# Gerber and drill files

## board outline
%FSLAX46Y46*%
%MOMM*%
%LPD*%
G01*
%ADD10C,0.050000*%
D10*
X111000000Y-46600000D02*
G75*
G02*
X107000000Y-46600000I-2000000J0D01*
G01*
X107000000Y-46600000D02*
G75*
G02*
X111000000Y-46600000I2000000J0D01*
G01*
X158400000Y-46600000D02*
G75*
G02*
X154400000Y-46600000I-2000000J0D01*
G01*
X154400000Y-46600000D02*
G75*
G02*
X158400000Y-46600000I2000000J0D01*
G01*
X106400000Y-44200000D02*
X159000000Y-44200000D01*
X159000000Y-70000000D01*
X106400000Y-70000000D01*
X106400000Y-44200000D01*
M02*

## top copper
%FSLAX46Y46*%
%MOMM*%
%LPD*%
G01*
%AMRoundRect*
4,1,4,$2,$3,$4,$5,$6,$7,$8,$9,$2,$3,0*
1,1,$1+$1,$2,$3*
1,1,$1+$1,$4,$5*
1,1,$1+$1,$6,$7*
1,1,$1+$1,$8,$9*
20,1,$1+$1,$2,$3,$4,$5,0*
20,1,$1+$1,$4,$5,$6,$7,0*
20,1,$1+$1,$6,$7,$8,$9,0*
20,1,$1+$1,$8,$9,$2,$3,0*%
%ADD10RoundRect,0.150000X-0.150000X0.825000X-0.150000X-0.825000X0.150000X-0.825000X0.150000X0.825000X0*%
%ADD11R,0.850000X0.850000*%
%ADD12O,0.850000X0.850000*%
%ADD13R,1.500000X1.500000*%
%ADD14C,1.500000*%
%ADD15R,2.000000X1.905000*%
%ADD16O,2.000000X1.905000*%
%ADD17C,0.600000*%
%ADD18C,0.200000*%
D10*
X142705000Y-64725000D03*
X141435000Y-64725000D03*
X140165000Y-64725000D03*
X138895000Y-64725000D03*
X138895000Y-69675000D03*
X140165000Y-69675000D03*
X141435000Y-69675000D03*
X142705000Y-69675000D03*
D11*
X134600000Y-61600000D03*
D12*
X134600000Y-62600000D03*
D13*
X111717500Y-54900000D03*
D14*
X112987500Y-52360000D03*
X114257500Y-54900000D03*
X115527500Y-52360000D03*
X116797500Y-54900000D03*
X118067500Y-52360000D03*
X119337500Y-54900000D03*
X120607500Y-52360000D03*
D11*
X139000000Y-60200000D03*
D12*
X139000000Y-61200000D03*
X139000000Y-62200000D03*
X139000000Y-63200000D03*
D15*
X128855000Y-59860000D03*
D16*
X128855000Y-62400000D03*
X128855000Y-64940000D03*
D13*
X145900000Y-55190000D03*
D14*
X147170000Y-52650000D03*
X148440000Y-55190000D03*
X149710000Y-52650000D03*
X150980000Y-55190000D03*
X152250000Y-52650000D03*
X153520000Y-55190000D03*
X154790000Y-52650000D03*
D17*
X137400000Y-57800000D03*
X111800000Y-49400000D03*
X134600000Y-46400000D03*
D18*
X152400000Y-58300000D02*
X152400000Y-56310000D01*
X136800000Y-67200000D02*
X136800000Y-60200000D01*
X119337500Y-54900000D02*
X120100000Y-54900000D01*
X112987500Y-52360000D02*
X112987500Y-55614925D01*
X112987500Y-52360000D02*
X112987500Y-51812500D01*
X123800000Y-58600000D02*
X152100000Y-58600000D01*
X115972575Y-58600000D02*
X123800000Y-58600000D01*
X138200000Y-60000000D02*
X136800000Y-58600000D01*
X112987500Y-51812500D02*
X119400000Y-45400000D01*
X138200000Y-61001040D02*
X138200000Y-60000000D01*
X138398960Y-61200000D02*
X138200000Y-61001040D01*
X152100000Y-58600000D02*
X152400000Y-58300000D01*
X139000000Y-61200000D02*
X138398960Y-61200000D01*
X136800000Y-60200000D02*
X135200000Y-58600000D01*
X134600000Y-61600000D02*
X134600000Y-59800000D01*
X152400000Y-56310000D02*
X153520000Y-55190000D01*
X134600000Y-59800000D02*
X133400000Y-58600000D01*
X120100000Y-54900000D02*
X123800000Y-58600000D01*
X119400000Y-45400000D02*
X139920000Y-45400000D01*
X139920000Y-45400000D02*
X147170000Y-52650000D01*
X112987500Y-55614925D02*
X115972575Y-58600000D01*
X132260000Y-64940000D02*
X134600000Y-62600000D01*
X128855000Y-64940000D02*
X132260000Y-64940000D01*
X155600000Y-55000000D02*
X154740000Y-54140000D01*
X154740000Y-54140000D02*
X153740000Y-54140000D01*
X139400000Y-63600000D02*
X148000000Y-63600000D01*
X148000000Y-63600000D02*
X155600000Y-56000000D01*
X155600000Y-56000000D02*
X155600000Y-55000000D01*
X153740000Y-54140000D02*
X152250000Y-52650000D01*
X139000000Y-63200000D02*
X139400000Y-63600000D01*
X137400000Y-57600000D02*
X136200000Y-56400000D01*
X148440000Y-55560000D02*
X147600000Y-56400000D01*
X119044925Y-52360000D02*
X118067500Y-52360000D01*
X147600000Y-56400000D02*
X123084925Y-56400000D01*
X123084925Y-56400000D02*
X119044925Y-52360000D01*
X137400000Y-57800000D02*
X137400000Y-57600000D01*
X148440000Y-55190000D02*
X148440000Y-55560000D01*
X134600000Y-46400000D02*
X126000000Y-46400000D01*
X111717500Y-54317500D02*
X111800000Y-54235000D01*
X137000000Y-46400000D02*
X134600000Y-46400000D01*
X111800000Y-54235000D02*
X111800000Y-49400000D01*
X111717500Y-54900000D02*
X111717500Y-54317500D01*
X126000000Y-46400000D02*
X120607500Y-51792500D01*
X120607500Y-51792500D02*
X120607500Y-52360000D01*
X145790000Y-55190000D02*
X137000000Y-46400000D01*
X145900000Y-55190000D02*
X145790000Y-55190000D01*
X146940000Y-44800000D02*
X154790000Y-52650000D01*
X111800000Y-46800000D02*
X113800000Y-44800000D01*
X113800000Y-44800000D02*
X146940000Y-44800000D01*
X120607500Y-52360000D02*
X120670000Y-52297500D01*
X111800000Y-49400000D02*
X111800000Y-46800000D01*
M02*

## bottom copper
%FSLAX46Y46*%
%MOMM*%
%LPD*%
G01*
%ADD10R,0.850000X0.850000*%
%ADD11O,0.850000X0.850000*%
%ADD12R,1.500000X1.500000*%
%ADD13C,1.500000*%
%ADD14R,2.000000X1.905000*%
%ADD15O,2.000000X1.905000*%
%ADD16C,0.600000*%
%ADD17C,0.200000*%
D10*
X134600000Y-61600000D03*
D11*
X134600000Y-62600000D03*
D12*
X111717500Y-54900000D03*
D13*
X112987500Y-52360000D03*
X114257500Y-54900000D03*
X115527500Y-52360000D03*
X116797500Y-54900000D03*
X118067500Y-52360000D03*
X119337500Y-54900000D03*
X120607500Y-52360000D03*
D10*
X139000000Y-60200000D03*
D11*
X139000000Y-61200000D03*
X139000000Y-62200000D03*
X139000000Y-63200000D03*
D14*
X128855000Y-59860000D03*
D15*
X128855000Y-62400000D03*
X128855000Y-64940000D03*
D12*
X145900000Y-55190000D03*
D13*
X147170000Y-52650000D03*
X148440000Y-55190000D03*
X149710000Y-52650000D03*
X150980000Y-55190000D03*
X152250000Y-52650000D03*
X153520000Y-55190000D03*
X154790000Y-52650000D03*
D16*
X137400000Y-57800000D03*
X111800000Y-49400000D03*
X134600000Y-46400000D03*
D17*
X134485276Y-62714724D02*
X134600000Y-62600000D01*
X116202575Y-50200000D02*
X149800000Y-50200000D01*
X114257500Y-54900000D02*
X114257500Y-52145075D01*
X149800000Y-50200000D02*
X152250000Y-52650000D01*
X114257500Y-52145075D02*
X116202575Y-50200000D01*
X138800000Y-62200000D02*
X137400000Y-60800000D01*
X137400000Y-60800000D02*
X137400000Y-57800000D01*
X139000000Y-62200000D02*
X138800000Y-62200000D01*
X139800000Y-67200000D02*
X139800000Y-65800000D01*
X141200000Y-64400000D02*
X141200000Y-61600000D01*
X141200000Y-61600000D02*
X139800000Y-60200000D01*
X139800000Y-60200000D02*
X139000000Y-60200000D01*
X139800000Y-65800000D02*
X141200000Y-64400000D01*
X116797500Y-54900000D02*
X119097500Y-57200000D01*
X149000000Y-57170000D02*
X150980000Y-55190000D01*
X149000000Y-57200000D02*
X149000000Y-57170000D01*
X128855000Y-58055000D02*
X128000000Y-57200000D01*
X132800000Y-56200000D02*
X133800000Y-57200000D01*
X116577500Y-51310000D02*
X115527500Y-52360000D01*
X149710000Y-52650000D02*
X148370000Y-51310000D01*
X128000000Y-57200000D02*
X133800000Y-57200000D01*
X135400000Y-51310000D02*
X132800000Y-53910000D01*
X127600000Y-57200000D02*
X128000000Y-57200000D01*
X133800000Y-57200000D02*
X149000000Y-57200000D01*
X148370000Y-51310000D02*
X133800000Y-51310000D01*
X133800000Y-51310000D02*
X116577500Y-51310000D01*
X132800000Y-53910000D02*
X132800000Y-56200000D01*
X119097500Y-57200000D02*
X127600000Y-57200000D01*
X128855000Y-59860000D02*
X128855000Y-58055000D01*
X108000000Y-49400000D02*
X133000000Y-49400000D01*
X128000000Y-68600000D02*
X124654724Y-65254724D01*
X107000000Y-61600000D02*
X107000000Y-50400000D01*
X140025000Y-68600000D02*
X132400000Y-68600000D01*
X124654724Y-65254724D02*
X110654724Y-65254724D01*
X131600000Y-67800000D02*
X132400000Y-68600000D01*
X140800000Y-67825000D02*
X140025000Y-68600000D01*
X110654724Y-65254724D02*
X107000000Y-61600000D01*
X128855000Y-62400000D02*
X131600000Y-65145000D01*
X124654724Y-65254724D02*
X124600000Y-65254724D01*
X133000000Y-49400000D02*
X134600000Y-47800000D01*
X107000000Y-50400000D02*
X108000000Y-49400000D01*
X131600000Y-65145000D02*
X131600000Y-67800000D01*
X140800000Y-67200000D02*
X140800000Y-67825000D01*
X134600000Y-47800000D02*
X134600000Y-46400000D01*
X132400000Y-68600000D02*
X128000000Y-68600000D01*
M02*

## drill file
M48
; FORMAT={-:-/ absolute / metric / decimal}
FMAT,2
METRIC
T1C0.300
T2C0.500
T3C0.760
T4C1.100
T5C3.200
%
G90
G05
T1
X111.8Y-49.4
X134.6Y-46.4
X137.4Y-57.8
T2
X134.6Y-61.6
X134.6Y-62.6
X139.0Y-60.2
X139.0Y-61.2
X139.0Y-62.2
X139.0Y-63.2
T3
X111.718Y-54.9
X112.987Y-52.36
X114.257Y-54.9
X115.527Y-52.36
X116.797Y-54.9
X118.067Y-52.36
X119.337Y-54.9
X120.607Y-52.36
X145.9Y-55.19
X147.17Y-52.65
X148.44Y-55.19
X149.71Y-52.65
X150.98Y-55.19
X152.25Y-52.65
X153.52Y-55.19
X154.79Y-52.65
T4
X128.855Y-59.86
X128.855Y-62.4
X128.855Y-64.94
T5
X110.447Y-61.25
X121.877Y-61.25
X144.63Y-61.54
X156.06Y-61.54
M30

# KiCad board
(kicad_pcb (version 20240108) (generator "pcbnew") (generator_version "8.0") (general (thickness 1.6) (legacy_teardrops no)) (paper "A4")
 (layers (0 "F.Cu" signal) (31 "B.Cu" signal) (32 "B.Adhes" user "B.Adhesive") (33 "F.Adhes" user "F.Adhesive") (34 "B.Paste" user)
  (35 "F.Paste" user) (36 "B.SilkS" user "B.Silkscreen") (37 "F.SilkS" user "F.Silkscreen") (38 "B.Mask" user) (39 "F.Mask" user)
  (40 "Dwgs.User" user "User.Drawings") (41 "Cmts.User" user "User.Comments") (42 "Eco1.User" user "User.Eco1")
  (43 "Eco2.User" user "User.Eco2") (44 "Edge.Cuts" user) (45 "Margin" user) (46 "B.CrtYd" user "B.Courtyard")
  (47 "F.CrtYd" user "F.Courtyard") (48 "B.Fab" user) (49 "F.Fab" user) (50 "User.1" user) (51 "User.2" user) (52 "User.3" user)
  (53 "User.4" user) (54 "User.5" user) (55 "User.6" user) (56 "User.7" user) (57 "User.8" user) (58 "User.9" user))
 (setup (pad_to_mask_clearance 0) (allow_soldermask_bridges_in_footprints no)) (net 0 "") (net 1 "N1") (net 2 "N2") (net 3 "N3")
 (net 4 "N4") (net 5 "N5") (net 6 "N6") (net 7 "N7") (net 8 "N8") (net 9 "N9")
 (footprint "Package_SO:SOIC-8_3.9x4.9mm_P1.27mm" (layer "F.Cu") (at 140.8 67.2 -90)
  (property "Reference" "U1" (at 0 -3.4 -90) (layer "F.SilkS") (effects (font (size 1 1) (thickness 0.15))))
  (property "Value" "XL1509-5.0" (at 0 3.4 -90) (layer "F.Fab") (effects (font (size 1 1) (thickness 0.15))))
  (pad "1" smd roundrect (at -2.475 -1.905 270) (size 1.95 0.6) (layers "F.Cu" "F.Paste" "F.Mask") (roundrect_rratio 0.25) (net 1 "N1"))
  (pad "2" smd roundrect (at -2.475 -0.635 270) (size 1.95 0.6) (layers "F.Cu" "F.Paste" "F.Mask") (roundrect_rratio 0.25) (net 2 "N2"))
  (pad "3" smd roundrect (at -2.475 0.635 270) (size 1.95 0.6) (layers "F.Cu" "F.Paste" "F.Mask") (roundrect_rratio 0.25) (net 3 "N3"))
  (pad "4" smd roundrect (at -2.475 1.905 270) (size 1.95 0.6) (layers "F.Cu" "F.Paste" "F.Mask") (roundrect_rratio 0.25) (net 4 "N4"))
  (pad "5" smd roundrect (at 2.475 1.905 270) (size 1.95 0.6) (layers "F.Cu" "F.Paste" "F.Mask") (roundrect_rratio 0.25) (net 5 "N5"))
  (pad "6" smd roundrect (at 2.475 0.635 270) (size 1.95 0.6) (layers "F.Cu" "F.Paste" "F.Mask") (roundrect_rratio 0.25))
  (pad "7" smd roundrect (at 2.475 -0.635 270) (size 1.95 0.6) (layers "F.Cu" "F.Paste" "F.Mask") (roundrect_rratio 0.25))
  (pad "8" smd roundrect (at 2.475 -1.905 270) (size 1.95 0.6) (layers "F.Cu" "F.Paste" "F.Mask") (roundrect_rratio 0.25)))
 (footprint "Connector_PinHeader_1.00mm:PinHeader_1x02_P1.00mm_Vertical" (layer "F.Cu") (at 134.6 61.6)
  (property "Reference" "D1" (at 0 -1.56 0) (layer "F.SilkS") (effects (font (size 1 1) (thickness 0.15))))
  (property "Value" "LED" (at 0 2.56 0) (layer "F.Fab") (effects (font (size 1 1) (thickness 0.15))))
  (pad "1" thru_hole rect (at 0 0) (size 0.85 0.85) (drill 0.5) (layers "*.Cu" "*.Mask") (remove_unused_layers no) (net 5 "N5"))
  (pad "2" thru_hole oval (at 0 1) (size 0.85 0.85) (drill 0.5) (layers "*.Cu" "*.Mask") (remove_unused_layers no) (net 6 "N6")))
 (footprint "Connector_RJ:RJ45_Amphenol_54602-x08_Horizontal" (layer "F.Cu") (at 111.7175 54.9)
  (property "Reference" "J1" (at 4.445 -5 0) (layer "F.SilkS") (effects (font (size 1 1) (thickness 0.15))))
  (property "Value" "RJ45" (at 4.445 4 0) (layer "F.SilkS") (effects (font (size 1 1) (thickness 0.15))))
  (pad "" np_thru_hole circle (at -1.27 6.35) (size 3.2 3.2) (drill 3.2) (layers "*.Cu" "*.Mask"))
  (pad "" np_thru_hole circle (at 10.16 6.35) (size 3.2 3.2) (drill 3.2) (layers "*.Cu" "*.Mask"))
  (pad "1" thru_hole rect (at 0 0) (size 1.5 1.5) (drill 0.76) (layers "*.Cu" "*.Mask") (remove_unused_layers no) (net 1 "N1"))
  (pad "2" thru_hole circle (at 1.27 -2.54) (size 1.5 1.5) (drill 0.76) (layers "*.Cu" "*.Mask") (remove_unused_layers no) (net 5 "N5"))
  (pad "3" thru_hole circle (at 2.54 0) (size 1.5 1.5) (drill 0.76) (layers "*.Cu" "*.Mask") (remove_unused_layers no) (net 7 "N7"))
  (pad "4" thru_hole circle (at 3.81 -2.54) (size 1.5 1.5) (drill 0.76) (layers "*.Cu" "*.Mask") (remove_unused_layers no) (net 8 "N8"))
  (pad "5" thru_hole circle (at 5.08 0) (size 1.5 1.5) (drill 0.76) (layers "*.Cu" "*.Mask") (remove_unused_layers no) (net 8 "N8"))
  (pad "6" thru_hole circle (at 6.35 -2.54) (size 1.5 1.5) (drill 0.76) (layers "*.Cu" "*.Mask") (remove_unused_layers no) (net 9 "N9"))
  (pad "7" thru_hole circle (at 7.62 0) (size 1.5 1.5) (drill 0.76) (layers "*.Cu" "*.Mask") (remove_unused_layers no) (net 5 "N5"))
  (pad "8" thru_hole circle (at 8.89 -2.54) (size 1.5 1.5) (drill 0.76) (layers "*.Cu" "*.Mask") (remove_unused_layers no) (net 1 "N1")))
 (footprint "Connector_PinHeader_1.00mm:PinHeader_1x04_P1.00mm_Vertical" (layer "F.Cu") (at 139 60.2)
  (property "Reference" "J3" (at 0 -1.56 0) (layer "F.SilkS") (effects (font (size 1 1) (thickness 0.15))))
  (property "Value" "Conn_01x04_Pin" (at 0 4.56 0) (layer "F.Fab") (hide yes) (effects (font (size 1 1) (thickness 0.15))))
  (pad "1" thru_hole rect (at 0 0) (size 0.85 0.85) (drill 0.5) (layers "*.Cu" "*.Mask") (remove_unused_layers no) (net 2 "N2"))
  (pad "2" thru_hole oval (at 0 1) (size 0.85 0.85) (drill 0.5) (layers "*.Cu" "*.Mask") (remove_unused_layers no) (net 5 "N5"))
  (pad "3" thru_hole oval (at 0 2) (size 0.85 0.85) (drill 0.5) (layers "*.Cu" "*.Mask") (remove_unused_layers no) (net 9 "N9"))
  (pad "4" thru_hole oval (at 0 3) (size 0.85 0.85) (drill 0.5) (layers "*.Cu" "*.Mask") (remove_unused_layers no) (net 7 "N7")))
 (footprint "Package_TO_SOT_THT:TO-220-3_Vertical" (layer "F.Cu") (at 128.855 59.86 -90)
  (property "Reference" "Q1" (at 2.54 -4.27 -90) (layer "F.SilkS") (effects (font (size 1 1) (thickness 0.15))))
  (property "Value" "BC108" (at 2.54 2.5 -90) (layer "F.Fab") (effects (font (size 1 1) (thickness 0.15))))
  (pad "1" thru_hole rect (at 0 0 270) (size 1.905 2) (drill 1.1) (layers "*.Cu" "*.Mask") (remove_unused_layers no) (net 8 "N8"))
  (pad "2" thru_hole oval (at 2.54 0 270) (size 1.905 2) (drill 1.1) (layers "*.Cu" "*.Mask") (remove_unused_layers no) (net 1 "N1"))
  (pad "3" thru_hole oval (at 5.08 0 270) (size 1.905 2) (drill 1.1) (layers "*.Cu" "*.Mask") (remove_unused_layers no) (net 6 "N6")))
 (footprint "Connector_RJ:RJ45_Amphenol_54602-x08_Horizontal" (layer "F.Cu") (at 145.9 55.19)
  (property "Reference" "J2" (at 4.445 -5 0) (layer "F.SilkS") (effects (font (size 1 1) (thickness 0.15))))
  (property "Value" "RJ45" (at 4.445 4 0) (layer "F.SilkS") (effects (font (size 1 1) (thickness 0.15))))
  (pad "" np_thru_hole circle (at -1.27 6.35) (size 3.2 3.2) (drill 3.2) (layers "*.Cu" "*.Mask"))
  (pad "" np_thru_hole circle (at 10.16 6.35) (size 3.2 3.2) (drill 3.2) (layers "*.Cu" "*.Mask"))
  (pad "1" thru_hole rect (at 0 0) (size 1.5 1.5) (drill 0.76) (layers "*.Cu" "*.Mask") (remove_unused_layers no) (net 1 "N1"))
  (pad "2" thru_hole circle (at 1.27 -2.54) (size 1.5 1.5) (drill 0.76) (layers "*.Cu" "*.Mask") (remove_unused_layers no) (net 5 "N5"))
  (pad "3" thru_hole circle (at 2.54 0) (size 1.5 1.5) (drill 0.76) (layers "*.Cu" "*.Mask") (remove_unused_layers no) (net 9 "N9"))
  (pad "4" thru_hole circle (at 3.81 -2.54) (size 1.5 1.5) (drill 0.76) (layers "*.Cu" "*.Mask") (remove_unused_layers no) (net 8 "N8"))
  (pad "5" thru_hole circle (at 5.08 0) (size 1.5 1.5) (drill 0.76) (layers "*.Cu" "*.Mask") (remove_unused_layers no) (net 8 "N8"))
  (pad "6" thru_hole circle (at 6.35 -2.54) (size 1.5 1.5) (drill 0.76) (layers "*.Cu" "*.Mask") (remove_unused_layers no) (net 7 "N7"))
  (pad "7" thru_hole circle (at 7.62 0) (size 1.5 1.5) (drill 0.76) (layers "*.Cu" "*.Mask") (remove_unused_layers no) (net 5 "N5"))
  (pad "8" thru_hole circle (at 8.89 -2.54) (size 1.5 1.5) (drill 0.76) (layers "*.Cu" "*.Mask") (remove_unused_layers no) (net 1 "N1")))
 (gr_circle (center 109 46.6) (end 110.6 47.8) (stroke (width 0.05) (type default)) (fill none) (layer "Edge.Cuts"))
 (gr_circle (center 156.4 46.6) (end 158 47.8) (stroke (width 0.05) (type default)) (fill none) (layer "Edge.Cuts"))
 (gr_rect (start 106.4 44.2) (end 159 70) (stroke (width 0.05) (type default)) (fill none) (layer "Edge.Cuts"))
 (segment (start 152.4 58.3) (end 152.4 56.31) (width 0.2) (layer "F.Cu") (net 5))
 (segment (start 136.8 67.2) (end 136.8 60.2) (width 0.2) (layer "F.Cu") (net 5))
 (segment (start 119.3375 54.9) (end 120.1 54.9) (width 0.2) (layer "F.Cu") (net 5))
 (segment (start 112.9875 52.36) (end 112.9875 55.614925) (width 0.2) (layer "F.Cu") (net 5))
 (segment (start 112.9875 52.36) (end 112.9875 51.8125) (width 0.2) (layer "F.Cu") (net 5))
 (segment (start 123.8 58.6) (end 152.1 58.6) (width 0.2) (layer "F.Cu") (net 5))
 (segment (start 115.972575 58.6) (end 123.8 58.6) (width 0.2) (layer "F.Cu") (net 5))
 (segment (start 138.2 60) (end 136.8 58.6) (width 0.2) (layer "F.Cu") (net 5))
 (segment (start 112.9875 51.8125) (end 119.4 45.4) (width 0.2) (layer "F.Cu") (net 5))
 (segment (start 138.2 61.00104) (end 138.2 60) (width 0.2) (layer "F.Cu") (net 5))
 (segment (start 138.39896 61.2) (end 138.2 61.00104) (width 0.2) (layer "F.Cu") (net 5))
 (segment (start 152.1 58.6) (end 152.4 58.3) (width 0.2) (layer "F.Cu") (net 5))
 (segment (start 139 61.2) (end 138.39896 61.2) (width 0.2) (layer "F.Cu") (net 5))
 (segment (start 136.8 60.2) (end 135.2 58.6) (width 0.2) (layer "F.Cu") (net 5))
 (segment (start 134.6 61.6) (end 134.6 59.8) (width 0.2) (layer "F.Cu") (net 5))
 (segment (start 152.4 56.31) (end 153.52 55.19) (width 0.2) (layer "F.Cu") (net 5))
 (segment (start 134.6 59.8) (end 133.4 58.6) (width 0.2) (layer "F.Cu") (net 5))
 (segment (start 120.1 54.9) (end 123.8 58.6) (width 0.2) (layer "F.Cu") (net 5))
 (segment (start 119.4 45.4) (end 139.92 45.4) (width 0.2) (layer "F.Cu") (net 5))
 (segment (start 139.92 45.4) (end 147.17 52.65) (width 0.2) (layer "F.Cu") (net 5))
 (segment (start 112.9875 55.614925) (end 115.972575 58.6) (width 0.2) (layer "F.Cu") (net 5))
 (segment (start 132.26 64.94) (end 134.6 62.6) (width 0.2) (layer "F.Cu") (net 6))
 (segment (start 128.855 64.94) (end 132.26 64.94) (width 0.2) (layer "F.Cu") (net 6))
 (segment (start 134.485276 62.714724) (end 134.6 62.6) (width 0.2) (layer "B.Cu") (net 6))
 (segment (start 155.6 55) (end 154.74 54.14) (width 0.2) (layer "F.Cu") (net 7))
 (segment (start 154.74 54.14) (end 153.74 54.14) (width 0.2) (layer "F.Cu") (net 7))
 (segment (start 139.4 63.6) (end 148 63.6) (width 0.2) (layer "F.Cu") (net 7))
 (segment (start 148 63.6) (end 155.6 56) (width 0.2) (layer "F.Cu") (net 7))
 (segment (start 155.6 56) (end 155.6 55) (width 0.2) (layer "F.Cu") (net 7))
 (segment (start 153.74 54.14) (end 152.25 52.65) (width 0.2) (layer "F.Cu") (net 7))
 (segment (start 139 63.2) (end 139.4 63.6) (width 0.2) (layer "F.Cu") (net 7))
 (segment (start 116.202575 50.2) (end 149.8 50.2) (width 0.2) (layer "B.Cu") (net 7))
 (segment (start 114.2575 54.9) (end 114.2575 52.145075) (width 0.2) (layer "B.Cu") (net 7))
 (segment (start 149.8 50.2) (end 152.25 52.65) (width 0.2) (layer "B.Cu") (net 7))
 (segment (start 114.2575 52.145075) (end 116.202575 50.2) (width 0.2) (layer "B.Cu") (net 7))
 (segment (start 137.4 57.6) (end 136.2 56.4) (width 0.2) (layer "F.Cu") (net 9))
 (segment (start 148.44 55.56) (end 147.6 56.4) (width 0.2) (layer "F.Cu") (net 9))
 (segment (start 119.044925 52.36) (end 118.0675 52.36) (width 0.2) (layer "F.Cu") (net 9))
 (segment (start 147.6 56.4) (end 123.084925 56.4) (width 0.2) (layer "F.Cu") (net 9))
 (segment (start 123.084925 56.4) (end 119.044925 52.36) (width 0.2) (layer "F.Cu") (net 9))
 (segment (start 137.4 57.8) (end 137.4 57.6) (width 0.2) (layer "F.Cu") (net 9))
 (segment (start 148.44 55.19) (end 148.44 55.56) (width 0.2) (layer "F.Cu") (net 9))
 (via (at 137.4 57.8) (size 0.6) (drill 0.3) (layers "F.Cu" "B.Cu") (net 9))
 (segment (start 138.8 62.2) (end 137.4 60.8) (width 0.2) (layer "B.Cu") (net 9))
 (segment (start 137.4 60.8) (end 137.4 57.8) (width 0.2) (layer "B.Cu") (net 9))
 (segment (start 139 62.2) (end 138.8 62.2) (width 0.2) (layer "B.Cu") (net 9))
 (segment (start 139.8 67.2) (end 139.8 65.8) (width 0.2) (layer "B.Cu") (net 2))
 (segment (start 141.2 64.4) (end 141.2 61.6) (width 0.2) (layer "B.Cu") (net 2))
 (segment (start 141.2 61.6) (end 139.8 60.2) (width 0.2) (layer "B.Cu") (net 2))
 (segment (start 139.8 60.2) (end 139 60.2) (width 0.2) (layer "B.Cu") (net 2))
 (segment (start 139.8 65.8) (end 141.2 64.4) (width 0.2) (layer "B.Cu") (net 2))
 (segment (start 116.7975 54.9) (end 119.0975 57.2) (width 0.2) (layer "B.Cu") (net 8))
 (segment (start 149 57.17) (end 150.98 55.19) (width 0.2) (layer "B.Cu") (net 8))
 (segment (start 149 57.2) (end 149 57.17) (width 0.2) (layer "B.Cu") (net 8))
 (segment (start 128.855 58.055) (end 128 57.2) (width 0.2) (layer "B.Cu") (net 8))
 (segment (start 132.8 56.2) (end 133.8 57.2) (width 0.2) (layer "B.Cu") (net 8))
 (segment (start 116.5775 51.31) (end 115.5275 52.36) (width 0.2) (layer "B.Cu") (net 8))
 (segment (start 149.71 52.65) (end 148.37 51.31) (width 0.2) (layer "B.Cu") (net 8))
 (segment (start 128 57.2) (end 133.8 57.2) (width 0.2) (layer "B.Cu") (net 8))
 (segment (start 135.4 51.31) (end 132.8 53.91) (width 0.2) (layer "B.Cu") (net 8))
 (segment (start 127.6 57.2) (end 128 57.2) (width 0.2) (layer "B.Cu") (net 8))
 (segment (start 133.8 57.2) (end 149 57.2) (width 0.2) (layer "B.Cu") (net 8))
 (segment (start 148.37 51.31) (end 133.8 51.31) (width 0.2) (layer "B.Cu") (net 8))
 (segment (start 133.8 51.31) (end 116.5775 51.31) (width 0.2) (layer "B.Cu") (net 8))
 (segment (start 132.8 53.91) (end 132.8 56.2) (width 0.2) (layer "B.Cu") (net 8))
 (segment (start 119.0975 57.2) (end 127.6 57.2) (width 0.2) (layer "B.Cu") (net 8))
 (segment (start 128.855 59.86) (end 128.855 58.055) (width 0.2) (layer "B.Cu") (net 8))
 (segment (start 134.6 46.4) (end 126 46.4) (width 0.2) (layer "F.Cu") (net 1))
 (segment (start 111.7175 54.3175) (end 111.8 54.235) (width 0.2) (layer "F.Cu") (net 1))
 (segment (start 137 46.4) (end 134.6 46.4) (width 0.2) (layer "F.Cu") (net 1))
 (segment (start 111.8 54.235) (end 111.8 49.4) (width 0.2) (layer "F.Cu") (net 1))
 (segment (start 111.7175 54.9) (end 111.7175 54.3175) (width 0.2) (layer "F.Cu") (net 1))
 (segment (start 126 46.4) (end 120.6075 51.7925) (width 0.2) (layer "F.Cu") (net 1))
 (segment (start 120.6075 51.7925) (end 120.6075 52.36) (width 0.2) (layer "F.Cu") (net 1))
 (segment (start 145.79 55.19) (end 137 46.4) (width 0.2) (layer "F.Cu") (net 1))
 (segment (start 145.9 55.19) (end 145.79 55.19) (width 0.2) (layer "F.Cu") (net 1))
 (segment (start 146.94 44.8) (end 154.79 52.65) (width 0.2) (layer "F.Cu") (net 1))
 (segment (start 111.8 46.8) (end 113.8 44.8) (width 0.2) (layer "F.Cu") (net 1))
 (segment (start 113.8 44.8) (end 146.94 44.8) (width 0.2) (layer "F.Cu") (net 1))
 (segment (start 120.6075 52.36) (end 120.67 52.2975) (width 0.2) (layer "F.Cu") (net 1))
 (segment (start 111.8 49.4) (end 111.8 46.8) (width 0.2) (layer "F.Cu") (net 1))
 (via (at 111.8 49.4) (size 0.6) (drill 0.3) (layers "F.Cu" "B.Cu") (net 1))
 (via (at 134.6 46.4) (size 0.6) (drill 0.3) (layers "F.Cu" "B.Cu") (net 1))
 (segment (start 108 49.4) (end 133 49.4) (width 0.2) (layer "B.Cu") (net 1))
 (segment (start 128 68.6) (end 124.654724 65.254724) (width 0.2) (layer "B.Cu") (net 1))
 (segment (start 107 61.6) (end 107 50.4) (width 0.2) (layer "B.Cu") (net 1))
 (segment (start 140.025 68.6) (end 132.4 68.6) (width 0.2) (layer "B.Cu") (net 1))
 (segment (start 124.654724 65.254724) (end 110.654724 65.254724) (width 0.2) (layer "B.Cu") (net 1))
 (segment (start 131.6 67.8) (end 132.4 68.6) (width 0.2) (layer "B.Cu") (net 1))
 (segment (start 140.8 67.825) (end 140.025 68.6) (width 0.2) (layer "B.Cu") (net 1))
 (segment (start 110.654724 65.254724) (end 107 61.6) (width 0.2) (layer "B.Cu") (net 1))
 (segment (start 128.855 62.4) (end 131.6 65.145) (width 0.2) (layer "B.Cu") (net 1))
 (segment (start 124.654724 65.254724) (end 124.6 65.254724) (width 0.2) (layer "B.Cu") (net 1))
 (segment (start 133 49.4) (end 134.6 47.8) (width 0.2) (layer "B.Cu") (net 1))
 (segment (start 107 50.4) (end 108 49.4) (width 0.2) (layer "B.Cu") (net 1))
 (segment (start 131.6 65.145) (end 131.6 67.8) (width 0.2) (layer "B.Cu") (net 1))
 (segment (start 140.8 67.2) (end 140.8 67.825) (width 0.2) (layer "B.Cu") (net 1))
 (segment (start 134.6 47.8) (end 134.6 46.4) (width 0.2) (layer "B.Cu") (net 1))
 (segment (start 132.4 68.6) (end 128 68.6) (width 0.2) (layer "B.Cu") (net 1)))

